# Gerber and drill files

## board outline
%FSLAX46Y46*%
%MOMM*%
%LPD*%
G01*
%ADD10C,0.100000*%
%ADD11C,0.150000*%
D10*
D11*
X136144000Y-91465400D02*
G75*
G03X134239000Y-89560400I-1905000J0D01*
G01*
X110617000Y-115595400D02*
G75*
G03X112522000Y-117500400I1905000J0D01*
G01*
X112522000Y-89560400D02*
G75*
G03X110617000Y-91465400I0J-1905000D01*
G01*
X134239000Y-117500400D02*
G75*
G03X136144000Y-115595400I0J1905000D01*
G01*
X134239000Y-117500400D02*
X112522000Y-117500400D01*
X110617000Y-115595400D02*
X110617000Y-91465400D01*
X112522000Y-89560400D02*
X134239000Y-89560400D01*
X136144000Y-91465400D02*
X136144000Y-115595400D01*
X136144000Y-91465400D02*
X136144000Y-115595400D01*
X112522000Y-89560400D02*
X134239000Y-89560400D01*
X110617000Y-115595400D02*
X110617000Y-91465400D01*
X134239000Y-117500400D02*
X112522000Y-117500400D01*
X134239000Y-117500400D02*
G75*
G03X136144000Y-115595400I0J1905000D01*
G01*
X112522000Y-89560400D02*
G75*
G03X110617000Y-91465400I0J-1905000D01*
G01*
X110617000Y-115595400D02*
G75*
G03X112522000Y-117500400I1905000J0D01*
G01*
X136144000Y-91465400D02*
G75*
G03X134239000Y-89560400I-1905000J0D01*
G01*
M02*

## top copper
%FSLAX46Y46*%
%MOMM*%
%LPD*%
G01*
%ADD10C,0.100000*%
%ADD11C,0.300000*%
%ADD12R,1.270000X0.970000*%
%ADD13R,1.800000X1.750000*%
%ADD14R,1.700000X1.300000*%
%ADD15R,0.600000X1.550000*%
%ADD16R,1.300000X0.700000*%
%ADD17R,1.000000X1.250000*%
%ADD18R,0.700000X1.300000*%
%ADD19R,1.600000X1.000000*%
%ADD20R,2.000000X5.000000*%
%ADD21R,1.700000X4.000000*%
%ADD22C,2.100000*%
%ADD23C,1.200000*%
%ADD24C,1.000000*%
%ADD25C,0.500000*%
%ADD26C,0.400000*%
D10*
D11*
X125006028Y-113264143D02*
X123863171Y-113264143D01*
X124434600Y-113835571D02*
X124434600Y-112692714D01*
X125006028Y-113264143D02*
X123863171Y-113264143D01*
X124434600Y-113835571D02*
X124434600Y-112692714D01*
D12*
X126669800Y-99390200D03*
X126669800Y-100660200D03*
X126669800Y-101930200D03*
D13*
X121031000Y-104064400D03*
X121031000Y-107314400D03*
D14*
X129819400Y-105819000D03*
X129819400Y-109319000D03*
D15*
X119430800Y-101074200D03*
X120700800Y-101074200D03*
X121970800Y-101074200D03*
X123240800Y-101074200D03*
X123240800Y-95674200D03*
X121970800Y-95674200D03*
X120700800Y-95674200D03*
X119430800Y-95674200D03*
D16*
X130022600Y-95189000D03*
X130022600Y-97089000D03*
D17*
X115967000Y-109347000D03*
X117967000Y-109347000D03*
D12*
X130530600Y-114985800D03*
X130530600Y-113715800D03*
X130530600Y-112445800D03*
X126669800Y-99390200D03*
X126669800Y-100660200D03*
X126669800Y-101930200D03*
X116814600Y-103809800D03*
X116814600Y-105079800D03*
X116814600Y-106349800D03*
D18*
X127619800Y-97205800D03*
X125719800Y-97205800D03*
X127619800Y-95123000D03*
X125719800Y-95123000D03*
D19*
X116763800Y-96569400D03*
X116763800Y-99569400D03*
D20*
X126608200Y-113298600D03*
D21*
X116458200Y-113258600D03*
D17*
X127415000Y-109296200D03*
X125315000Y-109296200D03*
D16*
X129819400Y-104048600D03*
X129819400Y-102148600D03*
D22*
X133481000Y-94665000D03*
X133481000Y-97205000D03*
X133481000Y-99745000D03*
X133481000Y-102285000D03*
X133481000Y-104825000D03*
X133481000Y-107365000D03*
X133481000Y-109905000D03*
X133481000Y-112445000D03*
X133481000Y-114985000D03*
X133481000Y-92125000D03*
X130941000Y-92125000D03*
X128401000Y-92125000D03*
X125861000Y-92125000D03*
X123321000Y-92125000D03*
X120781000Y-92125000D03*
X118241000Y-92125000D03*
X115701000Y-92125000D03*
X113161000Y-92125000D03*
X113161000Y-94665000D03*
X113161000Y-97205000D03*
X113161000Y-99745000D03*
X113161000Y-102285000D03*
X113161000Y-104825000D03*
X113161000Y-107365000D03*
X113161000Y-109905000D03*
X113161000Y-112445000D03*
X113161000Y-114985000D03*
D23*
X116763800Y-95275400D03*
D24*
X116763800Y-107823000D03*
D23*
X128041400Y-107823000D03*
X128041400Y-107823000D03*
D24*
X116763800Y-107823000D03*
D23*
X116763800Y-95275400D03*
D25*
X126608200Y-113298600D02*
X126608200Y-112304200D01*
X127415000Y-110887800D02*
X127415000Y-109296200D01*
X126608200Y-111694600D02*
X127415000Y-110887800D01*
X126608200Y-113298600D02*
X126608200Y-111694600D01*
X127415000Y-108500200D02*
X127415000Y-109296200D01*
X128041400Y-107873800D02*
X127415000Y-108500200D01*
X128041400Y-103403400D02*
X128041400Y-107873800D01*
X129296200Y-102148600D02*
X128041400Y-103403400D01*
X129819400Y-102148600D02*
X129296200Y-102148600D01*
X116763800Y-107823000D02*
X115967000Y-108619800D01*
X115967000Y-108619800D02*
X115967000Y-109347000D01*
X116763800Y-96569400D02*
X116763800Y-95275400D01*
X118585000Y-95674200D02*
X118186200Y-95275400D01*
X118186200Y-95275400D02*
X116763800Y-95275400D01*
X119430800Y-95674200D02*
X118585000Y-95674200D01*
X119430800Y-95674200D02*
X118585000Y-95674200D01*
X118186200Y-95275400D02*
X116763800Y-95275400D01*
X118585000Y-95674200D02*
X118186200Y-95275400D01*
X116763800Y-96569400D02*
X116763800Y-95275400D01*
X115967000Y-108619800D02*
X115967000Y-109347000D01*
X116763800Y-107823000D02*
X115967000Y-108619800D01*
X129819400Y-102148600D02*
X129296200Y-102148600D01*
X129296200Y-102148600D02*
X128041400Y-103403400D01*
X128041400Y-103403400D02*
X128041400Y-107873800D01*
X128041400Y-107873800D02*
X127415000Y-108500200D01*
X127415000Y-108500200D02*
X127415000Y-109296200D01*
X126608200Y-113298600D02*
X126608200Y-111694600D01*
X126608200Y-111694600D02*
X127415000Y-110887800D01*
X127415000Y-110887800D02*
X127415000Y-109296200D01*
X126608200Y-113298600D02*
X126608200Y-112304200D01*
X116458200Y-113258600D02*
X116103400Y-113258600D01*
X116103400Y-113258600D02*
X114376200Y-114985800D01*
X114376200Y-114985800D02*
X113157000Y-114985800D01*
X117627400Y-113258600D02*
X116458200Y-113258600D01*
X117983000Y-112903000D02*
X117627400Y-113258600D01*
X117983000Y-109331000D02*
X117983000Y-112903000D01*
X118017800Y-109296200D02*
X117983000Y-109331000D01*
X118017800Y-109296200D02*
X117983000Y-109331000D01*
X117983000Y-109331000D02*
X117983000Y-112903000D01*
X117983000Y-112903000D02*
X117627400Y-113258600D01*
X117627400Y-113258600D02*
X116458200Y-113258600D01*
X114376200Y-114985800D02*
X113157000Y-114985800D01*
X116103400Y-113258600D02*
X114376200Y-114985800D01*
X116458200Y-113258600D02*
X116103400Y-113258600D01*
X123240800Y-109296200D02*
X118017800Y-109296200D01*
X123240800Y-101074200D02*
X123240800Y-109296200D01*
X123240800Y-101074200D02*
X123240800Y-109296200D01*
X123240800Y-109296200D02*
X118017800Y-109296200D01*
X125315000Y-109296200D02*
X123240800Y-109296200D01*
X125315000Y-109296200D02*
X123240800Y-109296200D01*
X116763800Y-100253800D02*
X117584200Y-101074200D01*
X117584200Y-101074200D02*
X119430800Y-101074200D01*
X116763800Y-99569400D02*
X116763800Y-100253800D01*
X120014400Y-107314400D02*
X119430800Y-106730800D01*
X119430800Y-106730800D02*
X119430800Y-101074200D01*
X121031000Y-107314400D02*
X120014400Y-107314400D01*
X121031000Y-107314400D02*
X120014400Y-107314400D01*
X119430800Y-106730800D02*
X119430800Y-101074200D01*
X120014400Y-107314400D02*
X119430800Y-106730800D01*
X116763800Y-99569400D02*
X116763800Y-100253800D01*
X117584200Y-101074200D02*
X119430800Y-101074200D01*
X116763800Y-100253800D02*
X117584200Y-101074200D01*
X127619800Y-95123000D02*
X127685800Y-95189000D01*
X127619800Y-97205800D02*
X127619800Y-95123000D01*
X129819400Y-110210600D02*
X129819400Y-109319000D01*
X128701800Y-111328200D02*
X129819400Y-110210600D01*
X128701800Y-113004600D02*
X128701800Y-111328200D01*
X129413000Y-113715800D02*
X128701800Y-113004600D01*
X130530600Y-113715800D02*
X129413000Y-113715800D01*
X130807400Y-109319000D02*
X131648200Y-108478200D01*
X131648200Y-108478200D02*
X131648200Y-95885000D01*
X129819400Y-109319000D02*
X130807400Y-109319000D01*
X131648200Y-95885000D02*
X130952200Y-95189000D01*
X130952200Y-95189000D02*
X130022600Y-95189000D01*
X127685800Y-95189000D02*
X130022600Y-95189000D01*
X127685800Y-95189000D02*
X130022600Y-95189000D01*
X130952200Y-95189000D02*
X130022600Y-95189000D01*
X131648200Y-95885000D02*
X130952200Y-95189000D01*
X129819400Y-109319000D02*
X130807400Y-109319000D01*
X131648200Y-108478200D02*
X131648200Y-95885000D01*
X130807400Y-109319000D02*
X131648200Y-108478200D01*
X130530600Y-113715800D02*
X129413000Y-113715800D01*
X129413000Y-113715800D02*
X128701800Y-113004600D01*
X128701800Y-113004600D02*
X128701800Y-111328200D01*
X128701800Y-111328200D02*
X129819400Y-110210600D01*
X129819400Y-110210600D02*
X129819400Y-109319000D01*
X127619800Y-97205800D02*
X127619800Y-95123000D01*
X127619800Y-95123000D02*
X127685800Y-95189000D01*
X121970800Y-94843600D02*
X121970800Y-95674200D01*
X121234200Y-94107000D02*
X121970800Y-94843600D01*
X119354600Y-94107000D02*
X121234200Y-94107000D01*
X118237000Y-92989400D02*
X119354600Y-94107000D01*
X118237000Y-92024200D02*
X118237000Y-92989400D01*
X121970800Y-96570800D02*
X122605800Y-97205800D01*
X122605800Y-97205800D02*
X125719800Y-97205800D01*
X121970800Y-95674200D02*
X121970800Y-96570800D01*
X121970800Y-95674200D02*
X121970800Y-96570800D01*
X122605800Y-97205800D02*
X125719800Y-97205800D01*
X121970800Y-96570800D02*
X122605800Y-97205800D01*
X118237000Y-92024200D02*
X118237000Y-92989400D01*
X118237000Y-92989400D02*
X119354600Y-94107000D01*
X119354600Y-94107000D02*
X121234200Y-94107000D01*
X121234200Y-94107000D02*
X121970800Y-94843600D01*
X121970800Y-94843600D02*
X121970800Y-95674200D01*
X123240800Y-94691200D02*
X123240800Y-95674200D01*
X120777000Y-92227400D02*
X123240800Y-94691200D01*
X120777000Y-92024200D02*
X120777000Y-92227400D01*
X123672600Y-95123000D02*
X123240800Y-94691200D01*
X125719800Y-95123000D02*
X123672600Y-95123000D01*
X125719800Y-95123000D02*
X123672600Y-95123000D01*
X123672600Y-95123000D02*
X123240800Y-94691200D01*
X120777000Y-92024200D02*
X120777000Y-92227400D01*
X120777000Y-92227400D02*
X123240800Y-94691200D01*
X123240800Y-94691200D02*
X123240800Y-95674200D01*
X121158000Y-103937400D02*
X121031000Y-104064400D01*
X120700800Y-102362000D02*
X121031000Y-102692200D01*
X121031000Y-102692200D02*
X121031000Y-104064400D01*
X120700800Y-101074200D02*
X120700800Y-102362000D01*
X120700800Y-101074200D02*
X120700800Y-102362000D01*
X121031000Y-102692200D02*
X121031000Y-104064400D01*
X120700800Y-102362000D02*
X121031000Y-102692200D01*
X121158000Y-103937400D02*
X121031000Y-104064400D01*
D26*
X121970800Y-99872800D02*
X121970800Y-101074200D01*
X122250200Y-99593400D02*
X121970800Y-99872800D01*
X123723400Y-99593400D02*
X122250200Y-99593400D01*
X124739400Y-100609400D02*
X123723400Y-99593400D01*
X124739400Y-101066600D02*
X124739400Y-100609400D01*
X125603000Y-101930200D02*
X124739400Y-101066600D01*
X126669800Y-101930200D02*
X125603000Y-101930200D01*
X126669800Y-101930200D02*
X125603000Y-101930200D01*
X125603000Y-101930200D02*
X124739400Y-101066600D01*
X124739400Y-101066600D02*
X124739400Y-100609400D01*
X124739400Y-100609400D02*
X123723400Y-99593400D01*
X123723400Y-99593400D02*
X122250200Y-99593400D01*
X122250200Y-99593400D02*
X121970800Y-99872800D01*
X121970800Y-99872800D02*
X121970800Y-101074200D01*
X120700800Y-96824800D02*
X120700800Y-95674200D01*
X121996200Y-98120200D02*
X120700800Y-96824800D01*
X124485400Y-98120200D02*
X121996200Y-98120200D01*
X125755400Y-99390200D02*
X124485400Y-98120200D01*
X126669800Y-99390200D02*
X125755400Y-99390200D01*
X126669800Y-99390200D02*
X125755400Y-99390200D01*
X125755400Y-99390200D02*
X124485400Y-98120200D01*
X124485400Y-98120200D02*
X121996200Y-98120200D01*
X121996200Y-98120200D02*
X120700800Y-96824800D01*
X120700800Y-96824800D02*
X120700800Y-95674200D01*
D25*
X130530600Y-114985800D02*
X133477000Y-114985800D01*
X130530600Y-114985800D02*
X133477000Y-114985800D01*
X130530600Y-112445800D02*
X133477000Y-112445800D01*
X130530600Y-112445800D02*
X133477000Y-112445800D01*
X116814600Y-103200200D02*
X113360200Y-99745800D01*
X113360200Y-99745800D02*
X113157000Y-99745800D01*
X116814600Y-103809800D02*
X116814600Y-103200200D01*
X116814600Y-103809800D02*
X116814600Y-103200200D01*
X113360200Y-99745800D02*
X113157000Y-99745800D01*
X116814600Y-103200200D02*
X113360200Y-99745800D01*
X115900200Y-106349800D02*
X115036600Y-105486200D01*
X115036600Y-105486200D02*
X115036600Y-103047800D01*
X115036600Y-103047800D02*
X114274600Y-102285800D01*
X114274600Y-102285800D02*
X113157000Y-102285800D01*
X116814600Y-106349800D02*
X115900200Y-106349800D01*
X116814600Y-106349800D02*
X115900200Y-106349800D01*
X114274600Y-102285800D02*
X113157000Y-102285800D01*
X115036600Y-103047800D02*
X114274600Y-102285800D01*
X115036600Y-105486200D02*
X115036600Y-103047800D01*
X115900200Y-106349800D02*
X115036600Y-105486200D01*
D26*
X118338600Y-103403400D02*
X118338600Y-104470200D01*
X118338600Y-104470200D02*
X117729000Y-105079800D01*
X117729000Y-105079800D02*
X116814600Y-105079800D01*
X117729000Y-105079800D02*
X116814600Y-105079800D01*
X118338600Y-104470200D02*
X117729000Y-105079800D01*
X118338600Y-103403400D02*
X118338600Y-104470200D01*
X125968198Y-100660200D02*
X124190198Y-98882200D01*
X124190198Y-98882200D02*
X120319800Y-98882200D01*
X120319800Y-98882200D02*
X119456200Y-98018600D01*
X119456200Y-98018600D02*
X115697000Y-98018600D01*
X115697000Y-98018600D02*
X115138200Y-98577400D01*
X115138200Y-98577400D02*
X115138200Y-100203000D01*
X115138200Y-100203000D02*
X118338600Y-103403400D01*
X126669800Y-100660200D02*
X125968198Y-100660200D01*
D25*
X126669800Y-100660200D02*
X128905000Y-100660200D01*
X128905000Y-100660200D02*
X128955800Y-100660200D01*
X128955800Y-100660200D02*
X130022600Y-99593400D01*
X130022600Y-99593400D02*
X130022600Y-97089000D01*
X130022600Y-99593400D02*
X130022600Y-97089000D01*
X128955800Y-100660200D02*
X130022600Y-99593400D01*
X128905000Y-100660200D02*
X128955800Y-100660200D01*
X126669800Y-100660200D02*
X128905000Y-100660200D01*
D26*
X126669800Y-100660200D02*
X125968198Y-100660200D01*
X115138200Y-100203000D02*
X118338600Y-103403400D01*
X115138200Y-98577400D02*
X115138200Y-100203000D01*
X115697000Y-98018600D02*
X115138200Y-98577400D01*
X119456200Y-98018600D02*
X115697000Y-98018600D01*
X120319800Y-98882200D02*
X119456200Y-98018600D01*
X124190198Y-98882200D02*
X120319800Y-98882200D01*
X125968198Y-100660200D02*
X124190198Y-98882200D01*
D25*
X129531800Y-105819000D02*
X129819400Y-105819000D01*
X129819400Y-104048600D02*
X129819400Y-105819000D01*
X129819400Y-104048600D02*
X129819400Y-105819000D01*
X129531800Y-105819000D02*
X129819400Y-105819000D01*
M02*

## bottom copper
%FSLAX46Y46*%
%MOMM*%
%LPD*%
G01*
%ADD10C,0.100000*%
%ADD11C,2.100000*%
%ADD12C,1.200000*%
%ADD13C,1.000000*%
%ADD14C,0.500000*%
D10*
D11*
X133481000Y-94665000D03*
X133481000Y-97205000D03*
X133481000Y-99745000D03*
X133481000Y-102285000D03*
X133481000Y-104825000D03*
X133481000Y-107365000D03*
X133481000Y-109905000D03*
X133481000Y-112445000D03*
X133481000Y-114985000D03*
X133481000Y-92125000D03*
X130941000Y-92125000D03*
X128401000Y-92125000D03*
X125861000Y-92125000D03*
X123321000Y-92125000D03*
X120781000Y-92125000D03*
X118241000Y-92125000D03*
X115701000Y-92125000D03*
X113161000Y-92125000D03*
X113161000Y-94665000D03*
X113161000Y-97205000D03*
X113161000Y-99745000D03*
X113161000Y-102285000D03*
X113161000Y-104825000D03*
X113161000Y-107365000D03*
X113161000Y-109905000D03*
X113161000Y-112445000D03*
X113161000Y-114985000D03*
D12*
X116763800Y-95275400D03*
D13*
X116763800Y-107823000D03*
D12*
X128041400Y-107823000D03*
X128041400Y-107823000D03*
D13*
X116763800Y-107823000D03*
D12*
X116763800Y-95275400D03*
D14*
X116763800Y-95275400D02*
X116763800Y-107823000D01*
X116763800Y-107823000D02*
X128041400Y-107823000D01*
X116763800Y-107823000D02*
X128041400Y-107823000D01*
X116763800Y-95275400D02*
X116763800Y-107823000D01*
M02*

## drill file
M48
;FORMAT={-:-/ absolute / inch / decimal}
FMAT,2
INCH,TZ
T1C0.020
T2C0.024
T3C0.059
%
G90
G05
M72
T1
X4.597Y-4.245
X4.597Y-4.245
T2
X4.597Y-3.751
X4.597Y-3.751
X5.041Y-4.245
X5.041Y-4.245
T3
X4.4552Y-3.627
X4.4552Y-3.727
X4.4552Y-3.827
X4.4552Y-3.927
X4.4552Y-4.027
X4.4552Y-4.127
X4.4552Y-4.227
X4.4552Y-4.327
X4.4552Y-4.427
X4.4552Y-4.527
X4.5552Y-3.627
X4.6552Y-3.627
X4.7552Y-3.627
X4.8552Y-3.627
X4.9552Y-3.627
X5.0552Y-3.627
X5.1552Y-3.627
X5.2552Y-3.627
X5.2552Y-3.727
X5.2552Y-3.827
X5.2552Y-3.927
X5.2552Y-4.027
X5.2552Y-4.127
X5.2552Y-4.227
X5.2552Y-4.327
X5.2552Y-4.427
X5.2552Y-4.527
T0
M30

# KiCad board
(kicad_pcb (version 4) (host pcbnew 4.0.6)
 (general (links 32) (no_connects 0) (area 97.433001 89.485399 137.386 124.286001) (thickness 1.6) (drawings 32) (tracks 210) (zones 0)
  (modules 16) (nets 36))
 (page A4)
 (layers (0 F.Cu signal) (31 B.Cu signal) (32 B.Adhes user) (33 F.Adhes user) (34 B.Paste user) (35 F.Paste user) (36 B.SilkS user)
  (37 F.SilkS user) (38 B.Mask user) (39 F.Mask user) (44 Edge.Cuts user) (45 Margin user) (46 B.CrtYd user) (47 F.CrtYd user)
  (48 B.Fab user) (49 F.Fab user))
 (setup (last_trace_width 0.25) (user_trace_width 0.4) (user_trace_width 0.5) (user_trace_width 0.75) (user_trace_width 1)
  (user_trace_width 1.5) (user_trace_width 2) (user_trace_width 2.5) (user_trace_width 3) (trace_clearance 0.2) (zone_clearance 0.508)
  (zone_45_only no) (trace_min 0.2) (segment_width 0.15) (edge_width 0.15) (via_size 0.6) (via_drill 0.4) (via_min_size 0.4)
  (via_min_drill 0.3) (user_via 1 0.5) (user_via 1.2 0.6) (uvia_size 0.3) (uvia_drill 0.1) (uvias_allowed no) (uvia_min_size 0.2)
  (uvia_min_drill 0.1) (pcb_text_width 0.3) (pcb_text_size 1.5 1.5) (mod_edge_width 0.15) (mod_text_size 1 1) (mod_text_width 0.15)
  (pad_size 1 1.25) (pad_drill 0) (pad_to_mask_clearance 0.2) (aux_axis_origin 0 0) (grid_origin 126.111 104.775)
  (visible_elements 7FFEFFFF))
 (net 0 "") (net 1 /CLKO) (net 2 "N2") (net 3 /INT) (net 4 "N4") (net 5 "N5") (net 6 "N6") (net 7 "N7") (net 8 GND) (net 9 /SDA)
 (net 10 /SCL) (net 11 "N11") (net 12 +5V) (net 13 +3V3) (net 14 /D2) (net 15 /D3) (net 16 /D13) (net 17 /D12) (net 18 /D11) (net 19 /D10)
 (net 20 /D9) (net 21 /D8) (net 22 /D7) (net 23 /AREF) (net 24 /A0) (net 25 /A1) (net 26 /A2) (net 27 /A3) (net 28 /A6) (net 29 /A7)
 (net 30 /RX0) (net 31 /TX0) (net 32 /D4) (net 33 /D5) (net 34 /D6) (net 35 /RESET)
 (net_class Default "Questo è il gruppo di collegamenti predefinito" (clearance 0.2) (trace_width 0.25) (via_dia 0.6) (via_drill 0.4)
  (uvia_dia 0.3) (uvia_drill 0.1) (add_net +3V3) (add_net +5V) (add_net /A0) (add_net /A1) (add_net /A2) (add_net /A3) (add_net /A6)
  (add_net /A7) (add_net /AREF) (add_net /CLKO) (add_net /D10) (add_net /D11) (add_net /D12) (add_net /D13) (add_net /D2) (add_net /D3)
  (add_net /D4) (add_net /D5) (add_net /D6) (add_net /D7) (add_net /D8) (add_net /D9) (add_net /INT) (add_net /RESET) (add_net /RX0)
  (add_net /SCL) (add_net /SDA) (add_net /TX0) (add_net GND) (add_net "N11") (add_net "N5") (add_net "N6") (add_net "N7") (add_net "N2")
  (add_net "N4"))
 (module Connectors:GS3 (layer F.Cu) (at 126.6698 100.6602)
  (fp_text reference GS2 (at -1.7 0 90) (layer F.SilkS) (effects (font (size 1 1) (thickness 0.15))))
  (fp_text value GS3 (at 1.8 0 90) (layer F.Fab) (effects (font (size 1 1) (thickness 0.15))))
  (pad 1 smd rect (at 0 -1.27) (size 1.27 0.97) (layers F.Cu F.Paste F.Mask) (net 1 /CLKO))
  (pad 2 smd rect (at 0 0) (size 1.27 0.97) (layers F.Cu F.Paste F.Mask) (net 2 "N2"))
  (pad 3 smd rect (at 0 1.27) (size 1.27 0.97) (layers F.Cu F.Paste F.Mask) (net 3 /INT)))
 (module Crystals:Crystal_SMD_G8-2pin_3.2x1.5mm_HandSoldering (layer F.Cu) (at 121.031 105.6894 270)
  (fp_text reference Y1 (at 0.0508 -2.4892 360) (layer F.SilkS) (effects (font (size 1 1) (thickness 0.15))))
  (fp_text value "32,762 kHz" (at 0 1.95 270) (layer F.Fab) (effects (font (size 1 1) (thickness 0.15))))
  (pad 1 smd rect (at -1.625 0 270) (size 1.75 1.8) (layers F.Cu F.Paste F.Mask) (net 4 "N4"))
  (pad 2 smd rect (at 1.625 0 270) (size 1.75 1.8) (layers F.Cu F.Paste F.Mask) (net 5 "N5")))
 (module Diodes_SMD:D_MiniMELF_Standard (layer F.Cu) (at 129.8194 107.569 270)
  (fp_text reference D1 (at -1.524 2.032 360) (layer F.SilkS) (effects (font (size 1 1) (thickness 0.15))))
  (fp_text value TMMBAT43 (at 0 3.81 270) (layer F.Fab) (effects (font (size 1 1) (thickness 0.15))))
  (pad 1 smd rect (at -1.75 0 270) (size 1.3 1.7) (layers F.Cu F.Paste F.Mask) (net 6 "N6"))
  (pad 2 smd rect (at 1.75 0 270) (size 1.3 1.7) (layers F.Cu F.Paste F.Mask) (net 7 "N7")))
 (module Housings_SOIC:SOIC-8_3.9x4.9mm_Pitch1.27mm (layer F.Cu) (at 121.3358 98.3742 90)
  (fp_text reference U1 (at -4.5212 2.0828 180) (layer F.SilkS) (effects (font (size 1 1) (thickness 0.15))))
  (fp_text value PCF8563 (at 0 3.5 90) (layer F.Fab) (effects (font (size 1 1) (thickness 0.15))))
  (pad 1 smd rect (at -2.7 -1.905 90) (size 1.55 0.6) (layers F.Cu F.Paste F.Mask) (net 5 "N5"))
  (pad 2 smd rect (at -2.7 -0.635 90) (size 1.55 0.6) (layers F.Cu F.Paste F.Mask) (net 4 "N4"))
  (pad 3 smd rect (at -2.7 0.635 90) (size 1.55 0.6) (layers F.Cu F.Paste F.Mask) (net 3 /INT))
  (pad 4 smd rect (at -2.7 1.905 90) (size 1.55 0.6) (layers F.Cu F.Paste F.Mask) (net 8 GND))
  (pad 5 smd rect (at 2.7 1.905 90) (size 1.55 0.6) (layers F.Cu F.Paste F.Mask) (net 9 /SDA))
  (pad 6 smd rect (at 2.7 0.635 90) (size 1.55 0.6) (layers F.Cu F.Paste F.Mask) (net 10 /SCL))
  (pad 7 smd rect (at 2.7 -0.635 90) (size 1.55 0.6) (layers F.Cu F.Paste F.Mask) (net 1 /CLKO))
  (pad 8 smd rect (at 2.7 -1.905 90) (size 1.55 0.6) (layers F.Cu F.Paste F.Mask) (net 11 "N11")))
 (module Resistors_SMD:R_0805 (layer F.Cu) (at 130.0226 96.139 270)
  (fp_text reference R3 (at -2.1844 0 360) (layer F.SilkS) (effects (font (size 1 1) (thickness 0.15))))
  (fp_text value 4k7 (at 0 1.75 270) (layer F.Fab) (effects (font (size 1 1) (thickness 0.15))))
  (pad 1 smd rect (at -0.95 0 270) (size 0.7 1.3) (layers F.Cu F.Paste F.Mask) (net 7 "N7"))
  (pad 2 smd rect (at 0.95 0 270) (size 0.7 1.3) (layers F.Cu F.Paste F.Mask) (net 2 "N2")))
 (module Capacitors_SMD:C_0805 (layer F.Cu) (at 116.967 109.347)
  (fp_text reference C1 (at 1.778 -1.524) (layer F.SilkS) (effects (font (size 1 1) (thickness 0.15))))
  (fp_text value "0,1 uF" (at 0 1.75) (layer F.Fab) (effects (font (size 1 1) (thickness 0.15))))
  (pad 1 smd rect (at -1 0) (size 1 1.25) (layers F.Cu F.Paste F.Mask) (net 11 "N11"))
  (pad 2 smd rect (at 1 0) (size 1 1.25) (layers F.Cu F.Paste F.Mask) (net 8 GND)))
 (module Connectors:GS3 (layer F.Cu) (at 130.5306 113.7158 180)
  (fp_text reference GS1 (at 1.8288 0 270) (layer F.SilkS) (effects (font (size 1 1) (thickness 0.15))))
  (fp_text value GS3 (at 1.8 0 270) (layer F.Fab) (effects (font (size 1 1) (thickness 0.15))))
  (pad 1 smd rect (at 0 -1.27 180) (size 1.27 0.97) (layers F.Cu F.Paste F.Mask) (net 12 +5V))
  (pad 2 smd rect (at 0 0 180) (size 1.27 0.97) (layers F.Cu F.Paste F.Mask) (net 7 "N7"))
  (pad 3 smd rect (at 0 1.27 180) (size 1.27 0.97) (layers F.Cu F.Paste F.Mask) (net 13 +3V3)))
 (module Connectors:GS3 (layer F.Cu) (at 126.6698 100.6602)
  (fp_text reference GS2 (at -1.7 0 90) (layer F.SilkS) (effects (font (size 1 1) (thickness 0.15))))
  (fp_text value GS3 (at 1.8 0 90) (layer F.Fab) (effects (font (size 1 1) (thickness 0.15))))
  (pad 1 smd rect (at 0 -1.27) (size 1.27 0.97) (layers F.Cu F.Paste F.Mask) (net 1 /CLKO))
  (pad 2 smd rect (at 0 0) (size 1.27 0.97) (layers F.Cu F.Paste F.Mask) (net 2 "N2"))
  (pad 3 smd rect (at 0 1.27) (size 1.27 0.97) (layers F.Cu F.Paste F.Mask) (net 3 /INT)))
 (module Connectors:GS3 (layer F.Cu) (at 116.8146 105.0798)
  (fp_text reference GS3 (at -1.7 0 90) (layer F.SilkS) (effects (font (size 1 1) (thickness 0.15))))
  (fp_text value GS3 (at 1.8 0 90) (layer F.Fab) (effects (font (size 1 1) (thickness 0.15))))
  (pad 1 smd rect (at 0 -1.27) (size 1.27 0.97) (layers F.Cu F.Paste F.Mask) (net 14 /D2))
  (pad 2 smd rect (at 0 0) (size 1.27 0.97) (layers F.Cu F.Paste F.Mask) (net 2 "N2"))
  (pad 3 smd rect (at 0 1.27) (size 1.27 0.97) (layers F.Cu F.Paste F.Mask) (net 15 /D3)))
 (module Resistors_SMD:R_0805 (layer F.Cu) (at 126.6698 97.2058 180)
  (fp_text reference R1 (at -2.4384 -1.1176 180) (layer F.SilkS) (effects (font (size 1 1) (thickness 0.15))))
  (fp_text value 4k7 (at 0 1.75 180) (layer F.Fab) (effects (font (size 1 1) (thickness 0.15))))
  (pad 1 smd rect (at -0.95 0 180) (size 0.7 1.3) (layers F.Cu F.Paste F.Mask) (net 7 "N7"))
  (pad 2 smd rect (at 0.95 0 180) (size 0.7 1.3) (layers F.Cu F.Paste F.Mask) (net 10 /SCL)))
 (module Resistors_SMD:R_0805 (layer F.Cu) (at 126.6698 95.123 180)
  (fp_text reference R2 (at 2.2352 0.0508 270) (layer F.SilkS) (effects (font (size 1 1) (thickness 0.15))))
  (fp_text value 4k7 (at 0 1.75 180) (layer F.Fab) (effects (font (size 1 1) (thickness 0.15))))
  (pad 1 smd rect (at -0.95 0 180) (size 0.7 1.3) (layers F.Cu F.Paste F.Mask) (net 7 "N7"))
  (pad 2 smd rect (at 0.95 0 180) (size 0.7 1.3) (layers F.Cu F.Paste F.Mask) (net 9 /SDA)))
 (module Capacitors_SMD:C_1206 (layer F.Cu) (at 116.7638 98.0694 270)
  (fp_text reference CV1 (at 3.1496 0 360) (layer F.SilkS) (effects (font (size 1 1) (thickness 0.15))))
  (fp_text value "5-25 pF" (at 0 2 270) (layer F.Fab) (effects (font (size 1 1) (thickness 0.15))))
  (pad 1 smd rect (at -1.5 0 270) (size 1 1.6) (layers F.Cu F.Paste F.Mask) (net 11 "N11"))
  (pad 2 smd rect (at 1.5 0 270) (size 1 1.6) (layers F.Cu F.Paste F.Mask) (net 5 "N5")))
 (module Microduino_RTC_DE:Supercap (layer F.Cu) (at 121.4882 113.2586 180)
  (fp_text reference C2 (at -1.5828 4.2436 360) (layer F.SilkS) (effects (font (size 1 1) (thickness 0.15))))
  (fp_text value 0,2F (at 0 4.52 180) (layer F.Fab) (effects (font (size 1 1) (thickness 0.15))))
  (pad 1 smd rect (at -5.12 -0.04 180) (size 2 5) (layers F.Cu F.Paste F.Mask) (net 11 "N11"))
  (pad 2 smd rect (at 5.03 0 180) (size 1.7 4) (layers F.Cu F.Mask) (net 8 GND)))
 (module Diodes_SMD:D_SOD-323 (layer F.Cu) (at 126.365 109.2962 180)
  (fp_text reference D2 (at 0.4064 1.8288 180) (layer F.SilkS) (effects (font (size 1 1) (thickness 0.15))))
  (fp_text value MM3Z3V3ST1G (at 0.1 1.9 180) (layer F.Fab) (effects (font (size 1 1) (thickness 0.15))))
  (pad 1 smd rect (at -1.05 0 180) (size 1 1.25) (layers F.Cu F.Paste F.Mask) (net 11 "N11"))
  (pad 2 smd rect (at 1.05 0 180) (size 1 1.25) (layers F.Cu F.Paste F.Mask) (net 8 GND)))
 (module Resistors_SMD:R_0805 (layer F.Cu) (at 129.8194 103.0986 90)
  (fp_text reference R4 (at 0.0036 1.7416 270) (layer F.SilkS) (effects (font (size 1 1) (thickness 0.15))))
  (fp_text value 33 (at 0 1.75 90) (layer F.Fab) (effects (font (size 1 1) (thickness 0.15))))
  (pad 1 smd rect (at -0.95 0 90) (size 0.7 1.3) (layers F.Cu F.Paste F.Mask) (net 6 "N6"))
  (pad 2 smd rect (at 0.95 0 90) (size 0.7 1.3) (layers F.Cu F.Paste F.Mask) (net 11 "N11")))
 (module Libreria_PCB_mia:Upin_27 (layer B.Cu) (at 133.481 114.985 180)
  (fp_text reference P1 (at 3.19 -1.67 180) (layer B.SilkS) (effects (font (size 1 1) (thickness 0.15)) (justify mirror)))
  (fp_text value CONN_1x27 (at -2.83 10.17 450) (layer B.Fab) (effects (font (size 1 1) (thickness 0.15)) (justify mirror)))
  (pad 9 thru_hole circle (at 0 20.32 180) (size 2.1 2.1) (drill 1.5) (layers *.Cu *.Mask) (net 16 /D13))
  (pad 8 thru_hole circle (at 0 17.78 180) (size 2.1 2.1) (drill 1.5) (layers *.Cu *.Mask) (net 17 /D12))
  (pad 7 thru_hole circle (at 0 15.24 180) (size 2.1 2.1) (drill 1.5) (layers *.Cu *.Mask) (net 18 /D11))
  (pad 6 thru_hole circle (at 0 12.7 180) (size 2.1 2.1) (drill 1.5) (layers *.Cu *.Mask) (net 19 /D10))
  (pad 5 thru_hole circle (at 0 10.16 180) (size 2.1 2.1) (drill 1.5) (layers *.Cu *.Mask) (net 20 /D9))
  (pad 4 thru_hole circle (at 0 7.62 180) (size 2.1 2.1) (drill 1.5) (layers *.Cu *.Mask) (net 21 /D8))
  (pad 3 thru_hole circle (at 0 5.08 180) (size 2.1 2.1) (drill 1.5) (layers *.Cu *.Mask) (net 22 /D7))
  (pad 2 thru_hole circle (at 0 2.54 180) (size 2.1 2.1) (drill 1.5) (layers *.Cu *.Mask) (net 13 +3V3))
  (pad 1 thru_hole circle (at 0 0 180) (size 2.1 2.1) (drill 1.5) (layers *.Cu *.Mask) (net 12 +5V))
  (pad 10 thru_hole circle (at 0 22.86 180) (size 2.1 2.1) (drill 1.5) (layers *.Cu *.Mask) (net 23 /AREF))
  (pad 11 thru_hole circle (at 2.54 22.86 180) (size 2.1 2.1) (drill 1.5) (layers *.Cu *.Mask) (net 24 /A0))
  (pad 12 thru_hole circle (at 5.08 22.86 180) (size 2.1 2.1) (drill 1.5) (layers *.Cu *.Mask) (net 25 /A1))
  (pad 13 thru_hole circle (at 7.62 22.86 180) (size 2.1 2.1) (drill 1.5) (layers *.Cu *.Mask) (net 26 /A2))
  (pad 14 thru_hole circle (at 10.16 22.86 180) (size 2.1 2.1) (drill 1.5) (layers *.Cu *.Mask) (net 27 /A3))
  (pad 15 thru_hole circle (at 12.7 22.86 180) (size 2.1 2.1) (drill 1.5) (layers *.Cu *.Mask) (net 9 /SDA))
  (pad 16 thru_hole circle (at 15.24 22.86 180) (size 2.1 2.1) (drill 1.5) (layers *.Cu *.Mask) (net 10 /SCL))
  (pad 17 thru_hole circle (at 17.78 22.86 180) (size 2.1 2.1) (drill 1.5) (layers *.Cu *.Mask) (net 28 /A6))
  (pad 18 thru_hole circle (at 20.32 22.86 180) (size 2.1 2.1) (drill 1.5) (layers *.Cu *.Mask) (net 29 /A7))
  (pad 19 thru_hole circle (at 20.32 20.32 180) (size 2.1 2.1) (drill 1.5) (layers *.Cu *.Mask) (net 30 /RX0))
  (pad 20 thru_hole circle (at 20.32 17.78 180) (size 2.1 2.1) (drill 1.5) (layers *.Cu *.Mask) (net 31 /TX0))
  (pad 21 thru_hole circle (at 20.32 15.24 180) (size 2.1 2.1) (drill 1.5) (layers *.Cu *.Mask) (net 14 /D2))
  (pad 22 thru_hole circle (at 20.32 12.7 180) (size 2.1 2.1) (drill 1.5) (layers *.Cu *.Mask) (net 15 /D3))
  (pad 23 thru_hole circle (at 20.32 10.16 180) (size 2.1 2.1) (drill 1.5) (layers *.Cu *.Mask) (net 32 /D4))
  (pad 24 thru_hole circle (at 20.32 7.62 180) (size 2.1 2.1) (drill 1.5) (layers *.Cu *.Mask) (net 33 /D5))
  (pad 25 thru_hole circle (at 20.32 5.08 180) (size 2.1 2.1) (drill 1.5) (layers *.Cu *.Mask) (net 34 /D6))
  (pad 26 thru_hole circle (at 20.32 2.54 180) (size 2.1 2.1) (drill 1.5) (layers *.Cu *.Mask) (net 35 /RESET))
  (pad 27 thru_hole circle (at 20.32 0 180) (size 2.1 2.1) (drill 1.5) (layers *.Cu *.Mask) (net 8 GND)))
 (gr_arc (start 134.239 91.4654) (end 134.239 89.5604) (angle 90) (layer Edge.Cuts) (width 0.15))
 (gr_arc (start 112.522 115.5954) (end 112.522 117.5004) (angle 90) (layer Edge.Cuts) (width 0.15))
 (gr_arc (start 112.522 91.4654) (end 110.617 91.4654) (angle 90) (layer Edge.Cuts) (width 0.15))
 (gr_arc (start 134.239 115.5954) (end 136.144 115.5954) (angle 90) (layer Edge.Cuts) (width 0.15))
 (gr_line (start 134.239 117.5004) (end 112.522 117.5004) (angle 90) (layer Edge.Cuts) (width 0.15))
 (gr_line (start 110.617 115.5954) (end 110.617 91.4654) (angle 90) (layer Edge.Cuts) (width 0.15))
 (gr_line (start 112.522 89.5604) (end 134.239 89.5604) (angle 90) (layer Edge.Cuts) (width 0.15))
 (gr_line (start 136.144 91.4654) (end 136.144 115.5954) (angle 90) (layer Edge.Cuts) (width 0.15))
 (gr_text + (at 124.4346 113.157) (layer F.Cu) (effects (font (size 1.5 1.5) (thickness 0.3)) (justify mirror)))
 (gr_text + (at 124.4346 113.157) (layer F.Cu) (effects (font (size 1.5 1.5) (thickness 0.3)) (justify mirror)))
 (gr_line (start 136.144 91.4654) (end 136.144 115.5954) (angle 90) (layer Edge.Cuts) (width 0.15))
 (gr_line (start 112.522 89.5604) (end 134.239 89.5604) (angle 90) (layer Edge.Cuts) (width 0.15))
 (gr_line (start 110.617 115.5954) (end 110.617 91.4654) (angle 90) (layer Edge.Cuts) (width 0.15))
 (gr_line (start 134.239 117.5004) (end 112.522 117.5004) (angle 90) (layer Edge.Cuts) (width 0.15))
 (gr_arc (start 134.239 115.5954) (end 136.144 115.5954) (angle 90) (layer Edge.Cuts) (width 0.15))
 (gr_arc (start 112.522 91.4654) (end 110.617 91.4654) (angle 90) (layer Edge.Cuts) (width 0.15))
 (gr_arc (start 112.522 115.5954) (end 112.522 117.5004) (angle 90) (layer Edge.Cuts) (width 0.15))
 (gr_arc (start 134.239 91.4654) (end 134.239 89.5604) (angle 90) (layer Edge.Cuts) (width 0.15))
 (segment (start 126.6082 113.2986) (end 126.6082 112.3042) (width 0.5) (layer F.Cu) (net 11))
 (segment (start 127.415 110.8878) (end 127.415 109.2962) (width 0.5) (layer F.Cu) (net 11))
 (segment (start 126.6082 111.6946) (end 127.415 110.8878) (width 0.5) (layer F.Cu) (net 11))
 (segment (start 126.6082 113.2986) (end 126.6082 111.6946) (width 0.5) (layer F.Cu) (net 11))
 (segment (start 127.415 108.5002) (end 127.415 109.2962) (width 0.5) (layer F.Cu) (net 11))
 (segment (start 128.0414 107.8738) (end 127.415 108.5002) (width 0.5) (layer F.Cu) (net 11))
 (segment (start 128.0414 103.4034) (end 128.0414 107.8738) (width 0.5) (layer F.Cu) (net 11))
 (segment (start 129.2962 102.1486) (end 128.0414 103.4034) (width 0.5) (layer F.Cu) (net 11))
 (segment (start 129.8194 102.1486) (end 129.2962 102.1486) (width 0.5) (layer F.Cu) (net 11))
 (via (at 116.7638 95.2754) (size 1.2) (drill 0.6) (layers F.Cu B.Cu) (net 11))
 (segment (start 116.7638 95.2754) (end 116.7638 107.823) (width 0.5) (layer B.Cu) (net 11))
 (via (at 116.7638 107.823) (size 1) (drill 0.5) (layers F.Cu B.Cu) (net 11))
 (segment (start 116.7638 107.823) (end 115.967 108.6198) (width 0.5) (layer F.Cu) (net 11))
 (segment (start 115.967 108.6198) (end 115.967 109.347) (width 0.5) (layer F.Cu) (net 11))
 (segment (start 116.7638 96.5694) (end 116.7638 95.2754) (width 0.5) (layer F.Cu) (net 11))
 (segment (start 118.585 95.6742) (end 118.1862 95.2754) (width 0.5) (layer F.Cu) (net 11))
 (segment (start 118.1862 95.2754) (end 116.7638 95.2754) (width 0.5) (layer F.Cu) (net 11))
 (segment (start 119.4308 95.6742) (end 118.585 95.6742) (width 0.5) (layer F.Cu) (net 11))
 (via (at 128.0414 107.823) (size 1.2) (drill 0.6) (layers F.Cu B.Cu) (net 11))
 (segment (start 116.7638 107.823) (end 128.0414 107.823) (width 0.5) (layer B.Cu) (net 11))
 (segment (start 116.7638 107.823) (end 128.0414 107.823) (width 0.5) (layer B.Cu) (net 11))
 (via (at 128.0414 107.823) (size 1.2) (drill 0.6) (layers F.Cu B.Cu) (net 11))
 (segment (start 119.4308 95.6742) (end 118.585 95.6742) (width 0.5) (layer F.Cu) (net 11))
 (segment (start 118.1862 95.2754) (end 116.7638 95.2754) (width 0.5) (layer F.Cu) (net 11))
 (segment (start 118.585 95.6742) (end 118.1862 95.2754) (width 0.5) (layer F.Cu) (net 11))
 (segment (start 116.7638 96.5694) (end 116.7638 95.2754) (width 0.5) (layer F.Cu) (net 11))
 (segment (start 115.967 108.6198) (end 115.967 109.347) (width 0.5) (layer F.Cu) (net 11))
 (segment (start 116.7638 107.823) (end 115.967 108.6198) (width 0.5) (layer F.Cu) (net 11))
 (via (at 116.7638 107.823) (size 1) (drill 0.5) (layers F.Cu B.Cu) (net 11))
 (segment (start 116.7638 95.2754) (end 116.7638 107.823) (width 0.5) (layer B.Cu) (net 11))
 (via (at 116.7638 95.2754) (size 1.2) (drill 0.6) (layers F.Cu B.Cu) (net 11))
 (segment (start 129.8194 102.1486) (end 129.2962 102.1486) (width 0.5) (layer F.Cu) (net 11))
 (segment (start 129.2962 102.1486) (end 128.0414 103.4034) (width 0.5) (layer F.Cu) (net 11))
 (segment (start 128.0414 103.4034) (end 128.0414 107.8738) (width 0.5) (layer F.Cu) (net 11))
 (segment (start 128.0414 107.8738) (end 127.415 108.5002) (width 0.5) (layer F.Cu) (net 11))
 (segment (start 127.415 108.5002) (end 127.415 109.2962) (width 0.5) (layer F.Cu) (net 11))
 (segment (start 126.6082 113.2986) (end 126.6082 111.6946) (width 0.5) (layer F.Cu) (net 11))
 (segment (start 126.6082 111.6946) (end 127.415 110.8878) (width 0.5) (layer F.Cu) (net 11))
 (segment (start 127.415 110.8878) (end 127.415 109.2962) (width 0.5) (layer F.Cu) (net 11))
 (segment (start 126.6082 113.2986) (end 126.6082 112.3042) (width 0.5) (layer F.Cu) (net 11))
 (segment (start 116.4582 113.2586) (end 116.1034 113.2586) (width 0.5) (layer F.Cu) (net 8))
 (segment (start 116.1034 113.2586) (end 114.3762 114.9858) (width 0.5) (layer F.Cu) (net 8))
 (segment (start 114.3762 114.9858) (end 113.157 114.9858) (width 0.5) (layer F.Cu) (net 8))
 (segment (start 117.6274 113.2586) (end 116.4582 113.2586) (width 0.5) (layer F.Cu) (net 8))
 (segment (start 117.983 112.903) (end 117.6274 113.2586) (width 0.5) (layer F.Cu) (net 8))
 (segment (start 117.983 109.331) (end 117.983 112.903) (width 0.5) (layer F.Cu) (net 8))
 (segment (start 118.0178 109.2962) (end 117.983 109.331) (width 0.5) (layer F.Cu) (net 8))
 (segment (start 118.0178 109.2962) (end 117.983 109.331) (width 0.5) (layer F.Cu) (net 8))
 (segment (start 117.983 109.331) (end 117.983 112.903) (width 0.5) (layer F.Cu) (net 8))
 (segment (start 117.983 112.903) (end 117.6274 113.2586) (width 0.5) (layer F.Cu) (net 8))
 (segment (start 117.6274 113.2586) (end 116.4582 113.2586) (width 0.5) (layer F.Cu) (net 8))
 (segment (start 114.3762 114.9858) (end 113.157 114.9858) (width 0.5) (layer F.Cu) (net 8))
 (segment (start 116.1034 113.2586) (end 114.3762 114.9858) (width 0.5) (layer F.Cu) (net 8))
 (segment (start 116.4582 113.2586) (end 116.1034 113.2586) (width 0.5) (layer F.Cu) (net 8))
 (segment (start 123.2408 109.2962) (end 118.0178 109.2962) (width 0.5) (layer F.Cu) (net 8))
 (segment (start 123.2408 101.0742) (end 123.2408 109.2962) (width 0.5) (layer F.Cu) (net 8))
 (segment (start 123.2408 101.0742) (end 123.2408 109.2962) (width 0.5) (layer F.Cu) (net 8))
 (segment (start 123.2408 109.2962) (end 118.0178 109.2962) (width 0.5) (layer F.Cu) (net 8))
 (segment (start 125.315 109.2962) (end 123.2408 109.2962) (width 0.5) (layer F.Cu) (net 8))
 (segment (start 125.315 109.2962) (end 123.2408 109.2962) (width 0.5) (layer F.Cu) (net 8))
 (segment (start 116.7638 100.2538) (end 117.5842 101.0742) (width 0.5) (layer F.Cu) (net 5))
 (segment (start 117.5842 101.0742) (end 119.4308 101.0742) (width 0.5) (layer F.Cu) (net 5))
 (segment (start 116.7638 99.5694) (end 116.7638 100.2538) (width 0.5) (layer F.Cu) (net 5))
 (segment (start 120.0144 107.3144) (end 119.4308 106.7308) (width 0.5) (layer F.Cu) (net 5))
 (segment (start 119.4308 106.7308) (end 119.4308 101.0742) (width 0.5) (layer F.Cu) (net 5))
 (segment (start 121.031 107.3144) (end 120.0144 107.3144) (width 0.5) (layer F.Cu) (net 5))
 (segment (start 121.031 107.3144) (end 120.0144 107.3144) (width 0.5) (layer F.Cu) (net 5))
 (segment (start 119.4308 106.7308) (end 119.4308 101.0742) (width 0.5) (layer F.Cu) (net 5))
 (segment (start 120.0144 107.3144) (end 119.4308 106.7308) (width 0.5) (layer F.Cu) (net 5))
 (segment (start 116.7638 99.5694) (end 116.7638 100.2538) (width 0.5) (layer F.Cu) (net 5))
 (segment (start 117.5842 101.0742) (end 119.4308 101.0742) (width 0.5) (layer F.Cu) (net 5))
 (segment (start 116.7638 100.2538) (end 117.5842 101.0742) (width 0.5) (layer F.Cu) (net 5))
 (segment (start 127.6198 95.123) (end 127.6858 95.189) (width 0.5) (layer F.Cu) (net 7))
 (segment (start 127.6198 97.2058) (end 127.6198 95.123) (width 0.5) (layer F.Cu) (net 7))
 (segment (start 129.8194 110.2106) (end 129.8194 109.319) (width 0.5) (layer F.Cu) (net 7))
 (segment (start 128.7018 111.3282) (end 129.8194 110.2106) (width 0.5) (layer F.Cu) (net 7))
 (segment (start 128.7018 113.0046) (end 128.7018 111.3282) (width 0.5) (layer F.Cu) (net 7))
 (segment (start 129.413 113.7158) (end 128.7018 113.0046) (width 0.5) (layer F.Cu) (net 7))
 (segment (start 130.5306 113.7158) (end 129.413 113.7158) (width 0.5) (layer F.Cu) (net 7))
 (segment (start 130.8074 109.319) (end 131.6482 108.4782) (width 0.5) (layer F.Cu) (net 7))
 (segment (start 131.6482 108.4782) (end 131.6482 95.885) (width 0.5) (layer F.Cu) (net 7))
 (segment (start 129.8194 109.319) (end 130.8074 109.319) (width 0.5) (layer F.Cu) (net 7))
 (segment (start 131.6482 95.885) (end 130.9522 95.189) (width 0.5) (layer F.Cu) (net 7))
 (segment (start 130.9522 95.189) (end 130.0226 95.189) (width 0.5) (layer F.Cu) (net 7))
 (segment (start 127.6858 95.189) (end 130.0226 95.189) (width 0.5) (layer F.Cu) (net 7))
 (segment (start 127.6858 95.189) (end 130.0226 95.189) (width 0.5) (layer F.Cu) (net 7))
 (segment (start 130.9522 95.189) (end 130.0226 95.189) (width 0.5) (layer F.Cu) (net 7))
 (segment (start 131.6482 95.885) (end 130.9522 95.189) (width 0.5) (layer F.Cu) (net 7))
 (segment (start 129.8194 109.319) (end 130.8074 109.319) (width 0.5) (layer F.Cu) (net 7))
 (segment (start 131.6482 108.4782) (end 131.6482 95.885) (width 0.5) (layer F.Cu) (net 7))
 (segment (start 130.8074 109.319) (end 131.6482 108.4782) (width 0.5) (layer F.Cu) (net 7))
 (segment (start 130.5306 113.7158) (end 129.413 113.7158) (width 0.5) (layer F.Cu) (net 7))
 (segment (start 129.413 113.7158) (end 128.7018 113.0046) (width 0.5) (layer F.Cu) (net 7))
 (segment (start 128.7018 113.0046) (end 128.7018 111.3282) (width 0.5) (layer F.Cu) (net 7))
 (segment (start 128.7018 111.3282) (end 129.8194 110.2106) (width 0.5) (layer F.Cu) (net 7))
 (segment (start 129.8194 110.2106) (end 129.8194 109.319) (width 0.5) (layer F.Cu) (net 7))
 (segment (start 127.6198 97.2058) (end 127.6198 95.123) (width 0.5) (layer F.Cu) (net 7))
 (segment (start 127.6198 95.123) (end 127.6858 95.189) (width 0.5) (layer F.Cu) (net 7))
 (segment (start 121.9708 94.8436) (end 121.9708 95.6742) (width 0.5) (layer F.Cu) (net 10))
 (segment (start 121.2342 94.107) (end 121.9708 94.8436) (width 0.5) (layer F.Cu) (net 10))
 (segment (start 119.3546 94.107) (end 121.2342 94.107) (width 0.5) (layer F.Cu) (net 10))
 (segment (start 118.237 92.9894) (end 119.3546 94.107) (width 0.5) (layer F.Cu) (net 10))
 (segment (start 118.237 92.0242) (end 118.237 92.9894) (width 0.5) (layer F.Cu) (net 10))
 (segment (start 121.9708 96.5708) (end 122.6058 97.2058) (width 0.5) (layer F.Cu) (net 10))
 (segment (start 122.6058 97.2058) (end 125.7198 97.2058) (width 0.5) (layer F.Cu) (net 10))
 (segment (start 121.9708 95.6742) (end 121.9708 96.5708) (width 0.5) (layer F.Cu) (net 10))
 (segment (start 121.9708 95.6742) (end 121.9708 96.5708) (width 0.5) (layer F.Cu) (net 10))
 (segment (start 122.6058 97.2058) (end 125.7198 97.2058) (width 0.5) (layer F.Cu) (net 10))
 (segment (start 121.9708 96.5708) (end 122.6058 97.2058) (width 0.5) (layer F.Cu) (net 10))
 (segment (start 118.237 92.0242) (end 118.237 92.9894) (width 0.5) (layer F.Cu) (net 10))
 (segment (start 118.237 92.9894) (end 119.3546 94.107) (width 0.5) (layer F.Cu) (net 10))
 (segment (start 119.3546 94.107) (end 121.2342 94.107) (width 0.5) (layer F.Cu) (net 10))
 (segment (start 121.2342 94.107) (end 121.9708 94.8436) (width 0.5) (layer F.Cu) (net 10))
 (segment (start 121.9708 94.8436) (end 121.9708 95.6742) (width 0.5) (layer F.Cu) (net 10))
 (segment (start 123.2408 94.6912) (end 123.2408 95.6742) (width 0.5) (layer F.Cu) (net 9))
 (segment (start 120.777 92.2274) (end 123.2408 94.6912) (width 0.5) (layer F.Cu) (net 9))
 (segment (start 120.777 92.0242) (end 120.777 92.2274) (width 0.5) (layer F.Cu) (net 9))
 (segment (start 123.6726 95.123) (end 123.2408 94.6912) (width 0.5) (layer F.Cu) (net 9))
 (segment (start 125.7198 95.123) (end 123.6726 95.123) (width 0.5) (layer F.Cu) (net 9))
 (segment (start 125.7198 95.123) (end 123.6726 95.123) (width 0.5) (layer F.Cu) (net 9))
 (segment (start 123.6726 95.123) (end 123.2408 94.6912) (width 0.5) (layer F.Cu) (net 9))
 (segment (start 120.777 92.0242) (end 120.777 92.2274) (width 0.5) (layer F.Cu) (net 9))
 (segment (start 120.777 92.2274) (end 123.2408 94.6912) (width 0.5) (layer F.Cu) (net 9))
 (segment (start 123.2408 94.6912) (end 123.2408 95.6742) (width 0.5) (layer F.Cu) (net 9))
 (segment (start 121.158 103.9374) (end 121.031 104.0644) (width 0.5) (layer F.Cu) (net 4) (status 30))
 (segment (start 120.7008 102.362) (end 121.031 102.6922) (width 0.5) (layer F.Cu) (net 4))
 (segment (start 121.031 102.6922) (end 121.031 104.0644) (width 0.5) (layer F.Cu) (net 4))
 (segment (start 120.7008 101.0742) (end 120.7008 102.362) (width 0.5) (layer F.Cu) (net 4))
 (segment (start 120.7008 101.0742) (end 120.7008 102.362) (width 0.5) (layer F.Cu) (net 4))
 (segment (start 121.031 102.6922) (end 121.031 104.0644) (width 0.5) (layer F.Cu) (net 4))
 (segment (start 120.7008 102.362) (end 121.031 102.6922) (width 0.5) (layer F.Cu) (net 4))
 (segment (start 121.158 103.9374) (end 121.031 104.0644) (width 0.5) (layer F.Cu) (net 4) (status 30))
 (segment (start 121.9708 99.8728) (end 121.9708 101.0742) (width 0.4) (layer F.Cu) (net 3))
 (segment (start 122.2502 99.5934) (end 121.9708 99.8728) (width 0.4) (layer F.Cu) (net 3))
 (segment (start 123.7234 99.5934) (end 122.2502 99.5934) (width 0.4) (layer F.Cu) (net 3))
 (segment (start 124.7394 100.6094) (end 123.7234 99.5934) (width 0.4) (layer F.Cu) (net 3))
 (segment (start 124.7394 101.0666) (end 124.7394 100.6094) (width 0.4) (layer F.Cu) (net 3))
 (segment (start 125.603 101.9302) (end 124.7394 101.0666) (width 0.4) (layer F.Cu) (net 3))
 (segment (start 126.6698 101.9302) (end 125.603 101.9302) (width 0.4) (layer F.Cu) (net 3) (status 10))
 (segment (start 126.6698 101.9302) (end 125.603 101.9302) (width 0.4) (layer F.Cu) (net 3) (status 10))
 (segment (start 125.603 101.9302) (end 124.7394 101.0666) (width 0.4) (layer F.Cu) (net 3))
 (segment (start 124.7394 101.0666) (end 124.7394 100.6094) (width 0.4) (layer F.Cu) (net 3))
 (segment (start 124.7394 100.6094) (end 123.7234 99.5934) (width 0.4) (layer F.Cu) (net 3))
 (segment (start 123.7234 99.5934) (end 122.2502 99.5934) (width 0.4) (layer F.Cu) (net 3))
 (segment (start 122.2502 99.5934) (end 121.9708 99.8728) (width 0.4) (layer F.Cu) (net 3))
 (segment (start 121.9708 99.8728) (end 121.9708 101.0742) (width 0.4) (layer F.Cu) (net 3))
 (segment (start 120.7008 96.8248) (end 120.7008 95.6742) (width 0.4) (layer F.Cu) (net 1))
 (segment (start 121.9962 98.1202) (end 120.7008 96.8248) (width 0.4) (layer F.Cu) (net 1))
 (segment (start 124.4854 98.1202) (end 121.9962 98.1202) (width 0.4) (layer F.Cu) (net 1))
 (segment (start 125.7554 99.3902) (end 124.4854 98.1202) (width 0.4) (layer F.Cu) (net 1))
 (segment (start 126.6698 99.3902) (end 125.7554 99.3902) (width 0.4) (layer F.Cu) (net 1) (status 10))
 (segment (start 126.6698 99.3902) (end 125.7554 99.3902) (width 0.4) (layer F.Cu) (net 1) (status 10))
 (segment (start 125.7554 99.3902) (end 124.4854 98.1202) (width 0.4) (layer F.Cu) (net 1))
 (segment (start 124.4854 98.1202) (end 121.9962 98.1202) (width 0.4) (layer F.Cu) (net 1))
 (segment (start 121.9962 98.1202) (end 120.7008 96.8248) (width 0.4) (layer F.Cu) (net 1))
 (segment (start 120.7008 96.8248) (end 120.7008 95.6742) (width 0.4) (layer F.Cu) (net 1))
 (segment (start 130.5306 114.9858) (end 133.477 114.9858) (width 0.5) (layer F.Cu) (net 12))
 (segment (start 130.5306 114.9858) (end 133.477 114.9858) (width 0.5) (layer F.Cu) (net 12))
 (segment (start 130.5306 112.4458) (end 133.477 112.4458) (width 0.5) (layer F.Cu) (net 13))
 (segment (start 130.5306 112.4458) (end 133.477 112.4458) (width 0.5) (layer F.Cu) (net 13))
 (segment (start 116.8146 103.2002) (end 113.3602 99.7458) (width 0.5) (layer F.Cu) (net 14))
 (segment (start 113.3602 99.7458) (end 113.157 99.7458) (width 0.5) (layer F.Cu) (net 14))
 (segment (start 116.8146 103.8098) (end 116.8146 103.2002) (width 0.5) (layer F.Cu) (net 14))
 (segment (start 116.8146 103.8098) (end 116.8146 103.2002) (width 0.5) (layer F.Cu) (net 14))
 (segment (start 113.3602 99.7458) (end 113.157 99.7458) (width 0.5) (layer F.Cu) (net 14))
 (segment (start 116.8146 103.2002) (end 113.3602 99.7458) (width 0.5) (layer F.Cu) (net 14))
 (segment (start 115.9002 106.3498) (end 115.0366 105.4862) (width 0.5) (layer F.Cu) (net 15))
 (segment (start 115.0366 105.4862) (end 115.0366 103.0478) (width 0.5) (layer F.Cu) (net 15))
 (segment (start 115.0366 103.0478) (end 114.2746 102.2858) (width 0.5) (layer F.Cu) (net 15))
 (segment (start 114.2746 102.2858) (end 113.157 102.2858) (width 0.5) (layer F.Cu) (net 15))
 (segment (start 116.8146 106.3498) (end 115.9002 106.3498) (width 0.5) (layer F.Cu) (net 15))
 (segment (start 116.8146 106.3498) (end 115.9002 106.3498) (width 0.5) (layer F.Cu) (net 15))
 (segment (start 114.2746 102.2858) (end 113.157 102.2858) (width 0.5) (layer F.Cu) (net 15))
 (segment (start 115.0366 103.0478) (end 114.2746 102.2858) (width 0.5) (layer F.Cu) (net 15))
 (segment (start 115.0366 105.4862) (end 115.0366 103.0478) (width 0.5) (layer F.Cu) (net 15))
 (segment (start 115.9002 106.3498) (end 115.0366 105.4862) (width 0.5) (layer F.Cu) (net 15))
 (segment (start 118.3386 103.4034) (end 118.3386 104.4702) (width 0.4) (layer F.Cu) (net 2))
 (segment (start 118.3386 104.4702) (end 117.729 105.0798) (width 0.4) (layer F.Cu) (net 2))
 (segment (start 117.729 105.0798) (end 116.8146 105.0798) (width 0.4) (layer F.Cu) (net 2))
 (segment (start 117.729 105.0798) (end 116.8146 105.0798) (width 0.4) (layer F.Cu) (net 2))
 (segment (start 118.3386 104.4702) (end 117.729 105.0798) (width 0.4) (layer F.Cu) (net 2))
 (segment (start 118.3386 103.4034) (end 118.3386 104.4702) (width 0.4) (layer F.Cu) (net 2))
 (segment (start 125.968198 100.6602) (end 124.190198 98.8822) (width 0.4) (layer F.Cu) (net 2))
 (segment (start 124.190198 98.8822) (end 120.3198 98.8822) (width 0.4) (layer F.Cu) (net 2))
 (segment (start 120.3198 98.8822) (end 119.4562 98.0186) (width 0.4) (layer F.Cu) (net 2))
 (segment (start 119.4562 98.0186) (end 115.697 98.0186) (width 0.4) (layer F.Cu) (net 2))
 (segment (start 115.697 98.0186) (end 115.1382 98.5774) (width 0.4) (layer F.Cu) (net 2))
 (segment (start 115.1382 98.5774) (end 115.1382 100.203) (width 0.4) (layer F.Cu) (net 2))
 (segment (start 115.1382 100.203) (end 118.3386 103.4034) (width 0.4) (layer F.Cu) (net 2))
 (segment (start 126.6698 100.6602) (end 125.968198 100.6602) (width 0.4) (layer F.Cu) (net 2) (status 10))
 (segment (start 126.6698 100.6602) (end 128.905 100.6602) (width 0.5) (layer F.Cu) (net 2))
 (segment (start 128.905 100.6602) (end 128.9558 100.6602) (width 0.5) (layer F.Cu) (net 2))
 (segment (start 128.9558 100.6602) (end 130.0226 99.5934) (width 0.5) (layer F.Cu) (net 2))
 (segment (start 130.0226 99.5934) (end 130.0226 97.089) (width 0.5) (layer F.Cu) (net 2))
 (segment (start 130.0226 99.5934) (end 130.0226 97.089) (width 0.5) (layer F.Cu) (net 2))
 (segment (start 128.9558 100.6602) (end 130.0226 99.5934) (width 0.5) (layer F.Cu) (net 2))
 (segment (start 128.905 100.6602) (end 128.9558 100.6602) (width 0.5) (layer F.Cu) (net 2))
 (segment (start 126.6698 100.6602) (end 128.905 100.6602) (width 0.5) (layer F.Cu) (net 2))
 (segment (start 126.6698 100.6602) (end 125.968198 100.6602) (width 0.4) (layer F.Cu) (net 2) (status 10))
 (segment (start 115.1382 100.203) (end 118.3386 103.4034) (width 0.4) (layer F.Cu) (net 2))
 (segment (start 115.1382 98.5774) (end 115.1382 100.203) (width 0.4) (layer F.Cu) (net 2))
 (segment (start 115.697 98.0186) (end 115.1382 98.5774) (width 0.4) (layer F.Cu) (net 2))
 (segment (start 119.4562 98.0186) (end 115.697 98.0186) (width 0.4) (layer F.Cu) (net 2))
 (segment (start 120.3198 98.8822) (end 119.4562 98.0186) (width 0.4) (layer F.Cu) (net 2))
 (segment (start 124.190198 98.8822) (end 120.3198 98.8822) (width 0.4) (layer F.Cu) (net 2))
 (segment (start 125.968198 100.6602) (end 124.190198 98.8822) (width 0.4) (layer F.Cu) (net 2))
 (segment (start 129.5318 105.819) (end 129.8194 105.819) (width 0.5) (layer F.Cu) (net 6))
 (segment (start 129.8194 104.0486) (end 129.8194 105.819) (width 0.5) (layer F.Cu) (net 6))
 (segment (start 129.8194 104.0486) (end 129.8194 105.819) (width 0.5) (layer F.Cu) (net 6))
 (segment (start 129.5318 105.819) (end 129.8194 105.819) (width 0.5) (layer F.Cu) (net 6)))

